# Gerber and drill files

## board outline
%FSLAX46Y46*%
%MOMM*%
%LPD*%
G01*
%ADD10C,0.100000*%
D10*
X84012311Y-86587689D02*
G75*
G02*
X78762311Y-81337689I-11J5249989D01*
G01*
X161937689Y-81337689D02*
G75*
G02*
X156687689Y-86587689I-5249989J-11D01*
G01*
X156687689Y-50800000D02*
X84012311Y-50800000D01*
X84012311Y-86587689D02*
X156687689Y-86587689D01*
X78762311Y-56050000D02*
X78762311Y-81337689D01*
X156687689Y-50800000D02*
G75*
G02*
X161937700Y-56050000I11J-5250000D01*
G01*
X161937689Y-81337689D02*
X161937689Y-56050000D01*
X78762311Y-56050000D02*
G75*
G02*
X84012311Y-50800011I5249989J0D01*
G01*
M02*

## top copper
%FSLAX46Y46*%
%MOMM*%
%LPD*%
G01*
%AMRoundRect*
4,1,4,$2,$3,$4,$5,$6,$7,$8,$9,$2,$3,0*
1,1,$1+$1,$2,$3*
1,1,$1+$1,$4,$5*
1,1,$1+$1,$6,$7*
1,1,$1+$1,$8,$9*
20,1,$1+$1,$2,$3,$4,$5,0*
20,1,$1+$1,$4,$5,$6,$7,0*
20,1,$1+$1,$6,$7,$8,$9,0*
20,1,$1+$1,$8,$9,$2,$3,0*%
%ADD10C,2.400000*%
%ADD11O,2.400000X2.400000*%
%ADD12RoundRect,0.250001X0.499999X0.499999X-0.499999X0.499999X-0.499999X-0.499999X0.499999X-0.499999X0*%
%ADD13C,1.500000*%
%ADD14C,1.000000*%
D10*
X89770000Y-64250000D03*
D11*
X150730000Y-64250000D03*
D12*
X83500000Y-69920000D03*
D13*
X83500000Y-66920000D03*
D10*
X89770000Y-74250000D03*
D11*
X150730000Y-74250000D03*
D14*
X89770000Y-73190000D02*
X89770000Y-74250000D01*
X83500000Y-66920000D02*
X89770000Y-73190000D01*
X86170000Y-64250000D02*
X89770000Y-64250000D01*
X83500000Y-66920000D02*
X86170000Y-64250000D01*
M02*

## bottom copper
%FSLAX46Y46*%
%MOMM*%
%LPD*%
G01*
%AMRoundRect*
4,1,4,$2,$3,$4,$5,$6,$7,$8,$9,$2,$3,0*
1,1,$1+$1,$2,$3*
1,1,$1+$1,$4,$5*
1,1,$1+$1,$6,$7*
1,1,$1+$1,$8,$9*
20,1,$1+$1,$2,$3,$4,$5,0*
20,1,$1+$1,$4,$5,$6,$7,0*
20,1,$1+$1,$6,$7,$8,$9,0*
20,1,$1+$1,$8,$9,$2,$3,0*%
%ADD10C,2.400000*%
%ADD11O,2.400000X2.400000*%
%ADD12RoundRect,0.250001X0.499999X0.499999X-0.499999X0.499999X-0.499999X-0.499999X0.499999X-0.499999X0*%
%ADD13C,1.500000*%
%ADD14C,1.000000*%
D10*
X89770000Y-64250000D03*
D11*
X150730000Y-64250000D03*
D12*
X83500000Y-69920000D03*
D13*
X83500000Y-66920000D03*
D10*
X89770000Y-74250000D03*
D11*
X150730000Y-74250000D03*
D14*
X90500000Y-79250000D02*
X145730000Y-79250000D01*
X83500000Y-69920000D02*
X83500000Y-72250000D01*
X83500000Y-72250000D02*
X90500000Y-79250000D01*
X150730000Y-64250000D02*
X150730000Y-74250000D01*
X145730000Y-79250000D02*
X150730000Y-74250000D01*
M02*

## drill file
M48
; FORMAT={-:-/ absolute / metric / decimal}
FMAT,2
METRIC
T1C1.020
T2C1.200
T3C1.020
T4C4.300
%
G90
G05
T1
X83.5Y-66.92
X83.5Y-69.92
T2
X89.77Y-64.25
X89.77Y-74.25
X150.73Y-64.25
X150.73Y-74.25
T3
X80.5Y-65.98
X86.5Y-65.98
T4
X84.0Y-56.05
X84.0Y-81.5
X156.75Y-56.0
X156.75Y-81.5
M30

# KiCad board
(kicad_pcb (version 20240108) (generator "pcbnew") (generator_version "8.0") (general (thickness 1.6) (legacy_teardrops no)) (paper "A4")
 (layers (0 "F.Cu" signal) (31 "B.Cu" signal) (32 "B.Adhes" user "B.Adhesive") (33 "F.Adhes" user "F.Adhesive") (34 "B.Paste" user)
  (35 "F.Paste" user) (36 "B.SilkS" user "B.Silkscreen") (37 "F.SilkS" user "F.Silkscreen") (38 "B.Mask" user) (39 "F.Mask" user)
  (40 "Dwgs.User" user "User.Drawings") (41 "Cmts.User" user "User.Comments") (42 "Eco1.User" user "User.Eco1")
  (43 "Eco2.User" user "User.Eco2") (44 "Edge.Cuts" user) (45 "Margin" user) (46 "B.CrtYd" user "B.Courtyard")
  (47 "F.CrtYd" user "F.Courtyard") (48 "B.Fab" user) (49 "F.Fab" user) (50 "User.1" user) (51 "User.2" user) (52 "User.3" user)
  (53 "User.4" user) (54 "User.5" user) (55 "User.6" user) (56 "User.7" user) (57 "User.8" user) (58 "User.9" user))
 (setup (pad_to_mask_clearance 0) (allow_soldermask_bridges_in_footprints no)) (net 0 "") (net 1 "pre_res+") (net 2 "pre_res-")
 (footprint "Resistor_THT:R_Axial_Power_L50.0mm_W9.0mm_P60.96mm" (layer "F.Cu") (at 89.77 64.25)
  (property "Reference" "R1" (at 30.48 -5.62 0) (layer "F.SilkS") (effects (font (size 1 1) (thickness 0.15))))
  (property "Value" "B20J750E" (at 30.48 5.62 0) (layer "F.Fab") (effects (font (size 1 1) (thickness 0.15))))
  (pad "1" thru_hole circle (at 0 0) (size 2.4 2.4) (drill 1.2) (layers "*.Cu" "*.Mask") (remove_unused_layers no) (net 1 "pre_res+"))
  (pad "2" thru_hole oval (at 60.96 0) (size 2.4 2.4) (drill 1.2) (layers "*.Cu" "*.Mask") (remove_unused_layers no) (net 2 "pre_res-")))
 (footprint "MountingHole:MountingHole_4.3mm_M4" (layer "F.Cu") (at 156.75 81.5)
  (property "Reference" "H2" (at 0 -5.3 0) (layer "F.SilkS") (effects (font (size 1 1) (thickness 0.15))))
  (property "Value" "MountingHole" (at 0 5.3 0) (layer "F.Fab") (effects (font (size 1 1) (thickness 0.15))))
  (pad "" np_thru_hole circle (at 0 0) (size 4.3 4.3) (drill 4.3) (layers "*.Cu" "*.Mask")))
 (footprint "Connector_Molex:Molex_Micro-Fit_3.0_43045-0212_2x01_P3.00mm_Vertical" (layer "F.Cu") (at 83.5 69.92 180)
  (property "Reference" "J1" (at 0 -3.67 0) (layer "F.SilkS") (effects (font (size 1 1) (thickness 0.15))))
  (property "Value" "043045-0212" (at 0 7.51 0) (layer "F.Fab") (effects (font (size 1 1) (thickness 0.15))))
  (pad "" np_thru_hole circle (at -3 3.94 180) (size 1.02 1.02) (drill 1.02) (layers "*.Cu" "*.Mask"))
  (pad "" np_thru_hole circle (at 3 3.94 180) (size 1.02 1.02) (drill 1.02) (layers "*.Cu" "*.Mask"))
  (pad "1" thru_hole roundrect (at 0 0 180) (size 1.5 1.5) (drill 1.02) (layers "*.Cu" "*.Mask") (remove_unused_layers no)
   (roundrect_rratio 0.166667) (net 2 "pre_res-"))
  (pad "2" thru_hole circle (at 0 3 180) (size 1.5 1.5) (drill 1.02) (layers "*.Cu" "*.Mask") (remove_unused_layers no) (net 1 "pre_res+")))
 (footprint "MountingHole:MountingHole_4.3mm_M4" (layer "F.Cu") (at 84 81.5)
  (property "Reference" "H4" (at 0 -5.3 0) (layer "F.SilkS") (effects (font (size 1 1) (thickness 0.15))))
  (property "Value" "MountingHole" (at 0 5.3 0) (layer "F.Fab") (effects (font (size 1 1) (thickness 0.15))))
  (pad "" np_thru_hole circle (at 0 0) (size 4.3 4.3) (drill 4.3) (layers "*.Cu" "*.Mask")))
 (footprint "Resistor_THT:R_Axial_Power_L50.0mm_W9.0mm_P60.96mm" (layer "F.Cu") (at 89.77 74.25)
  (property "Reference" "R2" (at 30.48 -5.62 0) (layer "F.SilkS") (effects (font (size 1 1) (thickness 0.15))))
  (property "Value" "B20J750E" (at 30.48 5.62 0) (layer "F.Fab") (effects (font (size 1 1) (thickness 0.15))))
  (pad "1" thru_hole circle (at 0 0) (size 2.4 2.4) (drill 1.2) (layers "*.Cu" "*.Mask") (remove_unused_layers no) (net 1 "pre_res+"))
  (pad "2" thru_hole oval (at 60.96 0) (size 2.4 2.4) (drill 1.2) (layers "*.Cu" "*.Mask") (remove_unused_layers no) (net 2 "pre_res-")))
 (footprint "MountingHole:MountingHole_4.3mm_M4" (layer "F.Cu") (at 84 56.05)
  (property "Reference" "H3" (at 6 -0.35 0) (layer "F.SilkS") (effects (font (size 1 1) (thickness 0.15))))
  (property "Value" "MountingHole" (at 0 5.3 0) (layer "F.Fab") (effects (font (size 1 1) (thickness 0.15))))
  (pad "" np_thru_hole circle (at 0 0) (size 4.3 4.3) (drill 4.3) (layers "*.Cu" "*.Mask")))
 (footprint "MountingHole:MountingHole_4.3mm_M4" (layer "F.Cu") (at 156.75 56)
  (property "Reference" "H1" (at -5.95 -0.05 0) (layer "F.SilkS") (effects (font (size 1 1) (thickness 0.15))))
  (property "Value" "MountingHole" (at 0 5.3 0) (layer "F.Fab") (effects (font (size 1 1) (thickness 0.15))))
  (pad "" np_thru_hole circle (at 0 0) (size 4.3 4.3) (drill 4.3) (layers "*.Cu" "*.Mask")))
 (gr_arc (start 84.012311 86.587689) (mid 80.3 85.05) (end 78.762311 81.337689) (stroke (width 0.1) (type default)) (layer "Edge.Cuts"))
 (gr_arc (start 161.937689 81.337689) (mid 160.4 85.05) (end 156.687689 86.587689) (stroke (width 0.1) (type default)) (layer "Edge.Cuts"))
 (gr_line (start 156.687689 50.8) (end 84.012311 50.8) (stroke (width 0.1) (type default)) (layer "Edge.Cuts"))
 (gr_line (start 84.012311 86.587689) (end 156.687689 86.587689) (stroke (width 0.1) (type default)) (layer "Edge.Cuts"))
 (gr_line (start 78.762311 56.05) (end 78.762311 81.337689) (stroke (width 0.1) (type default)) (layer "Edge.Cuts"))
 (gr_arc (start 156.687689 50.8) (mid 160.4 52.337689) (end 161.937689 56.05) (stroke (width 0.1) (type default)) (layer "Edge.Cuts"))
 (gr_line (start 161.937689 81.337689) (end 161.937689 56.05) (stroke (width 0.1) (type default)) (layer "Edge.Cuts"))
 (gr_arc (start 78.762311 56.05) (mid 80.3 52.337689) (end 84.012311 50.8) (stroke (width 0.1) (type default)) (layer "Edge.Cuts"))
 (segment (start 89.77 73.19) (end 89.77 74.25) (width 1) (layer "F.Cu") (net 1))
 (segment (start 83.5 66.92) (end 89.77 73.19) (width 1) (layer "F.Cu") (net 1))
 (segment (start 86.17 64.25) (end 89.77 64.25) (width 1) (layer "F.Cu") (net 1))
 (segment (start 83.5 66.92) (end 86.17 64.25) (width 1) (layer "F.Cu") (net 1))
 (segment (start 90.5 79.25) (end 145.73 79.25) (width 1) (layer "B.Cu") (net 2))
 (segment (start 83.5 69.92) (end 83.5 72.25) (width 1) (layer "B.Cu") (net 2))
 (segment (start 83.5 72.25) (end 90.5 79.25) (width 1) (layer "B.Cu") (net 2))
 (segment (start 150.73 64.25) (end 150.73 74.25) (width 1) (layer "B.Cu") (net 2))
 (segment (start 145.73 79.25) (end 150.73 74.25) (width 1) (layer "B.Cu") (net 2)))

